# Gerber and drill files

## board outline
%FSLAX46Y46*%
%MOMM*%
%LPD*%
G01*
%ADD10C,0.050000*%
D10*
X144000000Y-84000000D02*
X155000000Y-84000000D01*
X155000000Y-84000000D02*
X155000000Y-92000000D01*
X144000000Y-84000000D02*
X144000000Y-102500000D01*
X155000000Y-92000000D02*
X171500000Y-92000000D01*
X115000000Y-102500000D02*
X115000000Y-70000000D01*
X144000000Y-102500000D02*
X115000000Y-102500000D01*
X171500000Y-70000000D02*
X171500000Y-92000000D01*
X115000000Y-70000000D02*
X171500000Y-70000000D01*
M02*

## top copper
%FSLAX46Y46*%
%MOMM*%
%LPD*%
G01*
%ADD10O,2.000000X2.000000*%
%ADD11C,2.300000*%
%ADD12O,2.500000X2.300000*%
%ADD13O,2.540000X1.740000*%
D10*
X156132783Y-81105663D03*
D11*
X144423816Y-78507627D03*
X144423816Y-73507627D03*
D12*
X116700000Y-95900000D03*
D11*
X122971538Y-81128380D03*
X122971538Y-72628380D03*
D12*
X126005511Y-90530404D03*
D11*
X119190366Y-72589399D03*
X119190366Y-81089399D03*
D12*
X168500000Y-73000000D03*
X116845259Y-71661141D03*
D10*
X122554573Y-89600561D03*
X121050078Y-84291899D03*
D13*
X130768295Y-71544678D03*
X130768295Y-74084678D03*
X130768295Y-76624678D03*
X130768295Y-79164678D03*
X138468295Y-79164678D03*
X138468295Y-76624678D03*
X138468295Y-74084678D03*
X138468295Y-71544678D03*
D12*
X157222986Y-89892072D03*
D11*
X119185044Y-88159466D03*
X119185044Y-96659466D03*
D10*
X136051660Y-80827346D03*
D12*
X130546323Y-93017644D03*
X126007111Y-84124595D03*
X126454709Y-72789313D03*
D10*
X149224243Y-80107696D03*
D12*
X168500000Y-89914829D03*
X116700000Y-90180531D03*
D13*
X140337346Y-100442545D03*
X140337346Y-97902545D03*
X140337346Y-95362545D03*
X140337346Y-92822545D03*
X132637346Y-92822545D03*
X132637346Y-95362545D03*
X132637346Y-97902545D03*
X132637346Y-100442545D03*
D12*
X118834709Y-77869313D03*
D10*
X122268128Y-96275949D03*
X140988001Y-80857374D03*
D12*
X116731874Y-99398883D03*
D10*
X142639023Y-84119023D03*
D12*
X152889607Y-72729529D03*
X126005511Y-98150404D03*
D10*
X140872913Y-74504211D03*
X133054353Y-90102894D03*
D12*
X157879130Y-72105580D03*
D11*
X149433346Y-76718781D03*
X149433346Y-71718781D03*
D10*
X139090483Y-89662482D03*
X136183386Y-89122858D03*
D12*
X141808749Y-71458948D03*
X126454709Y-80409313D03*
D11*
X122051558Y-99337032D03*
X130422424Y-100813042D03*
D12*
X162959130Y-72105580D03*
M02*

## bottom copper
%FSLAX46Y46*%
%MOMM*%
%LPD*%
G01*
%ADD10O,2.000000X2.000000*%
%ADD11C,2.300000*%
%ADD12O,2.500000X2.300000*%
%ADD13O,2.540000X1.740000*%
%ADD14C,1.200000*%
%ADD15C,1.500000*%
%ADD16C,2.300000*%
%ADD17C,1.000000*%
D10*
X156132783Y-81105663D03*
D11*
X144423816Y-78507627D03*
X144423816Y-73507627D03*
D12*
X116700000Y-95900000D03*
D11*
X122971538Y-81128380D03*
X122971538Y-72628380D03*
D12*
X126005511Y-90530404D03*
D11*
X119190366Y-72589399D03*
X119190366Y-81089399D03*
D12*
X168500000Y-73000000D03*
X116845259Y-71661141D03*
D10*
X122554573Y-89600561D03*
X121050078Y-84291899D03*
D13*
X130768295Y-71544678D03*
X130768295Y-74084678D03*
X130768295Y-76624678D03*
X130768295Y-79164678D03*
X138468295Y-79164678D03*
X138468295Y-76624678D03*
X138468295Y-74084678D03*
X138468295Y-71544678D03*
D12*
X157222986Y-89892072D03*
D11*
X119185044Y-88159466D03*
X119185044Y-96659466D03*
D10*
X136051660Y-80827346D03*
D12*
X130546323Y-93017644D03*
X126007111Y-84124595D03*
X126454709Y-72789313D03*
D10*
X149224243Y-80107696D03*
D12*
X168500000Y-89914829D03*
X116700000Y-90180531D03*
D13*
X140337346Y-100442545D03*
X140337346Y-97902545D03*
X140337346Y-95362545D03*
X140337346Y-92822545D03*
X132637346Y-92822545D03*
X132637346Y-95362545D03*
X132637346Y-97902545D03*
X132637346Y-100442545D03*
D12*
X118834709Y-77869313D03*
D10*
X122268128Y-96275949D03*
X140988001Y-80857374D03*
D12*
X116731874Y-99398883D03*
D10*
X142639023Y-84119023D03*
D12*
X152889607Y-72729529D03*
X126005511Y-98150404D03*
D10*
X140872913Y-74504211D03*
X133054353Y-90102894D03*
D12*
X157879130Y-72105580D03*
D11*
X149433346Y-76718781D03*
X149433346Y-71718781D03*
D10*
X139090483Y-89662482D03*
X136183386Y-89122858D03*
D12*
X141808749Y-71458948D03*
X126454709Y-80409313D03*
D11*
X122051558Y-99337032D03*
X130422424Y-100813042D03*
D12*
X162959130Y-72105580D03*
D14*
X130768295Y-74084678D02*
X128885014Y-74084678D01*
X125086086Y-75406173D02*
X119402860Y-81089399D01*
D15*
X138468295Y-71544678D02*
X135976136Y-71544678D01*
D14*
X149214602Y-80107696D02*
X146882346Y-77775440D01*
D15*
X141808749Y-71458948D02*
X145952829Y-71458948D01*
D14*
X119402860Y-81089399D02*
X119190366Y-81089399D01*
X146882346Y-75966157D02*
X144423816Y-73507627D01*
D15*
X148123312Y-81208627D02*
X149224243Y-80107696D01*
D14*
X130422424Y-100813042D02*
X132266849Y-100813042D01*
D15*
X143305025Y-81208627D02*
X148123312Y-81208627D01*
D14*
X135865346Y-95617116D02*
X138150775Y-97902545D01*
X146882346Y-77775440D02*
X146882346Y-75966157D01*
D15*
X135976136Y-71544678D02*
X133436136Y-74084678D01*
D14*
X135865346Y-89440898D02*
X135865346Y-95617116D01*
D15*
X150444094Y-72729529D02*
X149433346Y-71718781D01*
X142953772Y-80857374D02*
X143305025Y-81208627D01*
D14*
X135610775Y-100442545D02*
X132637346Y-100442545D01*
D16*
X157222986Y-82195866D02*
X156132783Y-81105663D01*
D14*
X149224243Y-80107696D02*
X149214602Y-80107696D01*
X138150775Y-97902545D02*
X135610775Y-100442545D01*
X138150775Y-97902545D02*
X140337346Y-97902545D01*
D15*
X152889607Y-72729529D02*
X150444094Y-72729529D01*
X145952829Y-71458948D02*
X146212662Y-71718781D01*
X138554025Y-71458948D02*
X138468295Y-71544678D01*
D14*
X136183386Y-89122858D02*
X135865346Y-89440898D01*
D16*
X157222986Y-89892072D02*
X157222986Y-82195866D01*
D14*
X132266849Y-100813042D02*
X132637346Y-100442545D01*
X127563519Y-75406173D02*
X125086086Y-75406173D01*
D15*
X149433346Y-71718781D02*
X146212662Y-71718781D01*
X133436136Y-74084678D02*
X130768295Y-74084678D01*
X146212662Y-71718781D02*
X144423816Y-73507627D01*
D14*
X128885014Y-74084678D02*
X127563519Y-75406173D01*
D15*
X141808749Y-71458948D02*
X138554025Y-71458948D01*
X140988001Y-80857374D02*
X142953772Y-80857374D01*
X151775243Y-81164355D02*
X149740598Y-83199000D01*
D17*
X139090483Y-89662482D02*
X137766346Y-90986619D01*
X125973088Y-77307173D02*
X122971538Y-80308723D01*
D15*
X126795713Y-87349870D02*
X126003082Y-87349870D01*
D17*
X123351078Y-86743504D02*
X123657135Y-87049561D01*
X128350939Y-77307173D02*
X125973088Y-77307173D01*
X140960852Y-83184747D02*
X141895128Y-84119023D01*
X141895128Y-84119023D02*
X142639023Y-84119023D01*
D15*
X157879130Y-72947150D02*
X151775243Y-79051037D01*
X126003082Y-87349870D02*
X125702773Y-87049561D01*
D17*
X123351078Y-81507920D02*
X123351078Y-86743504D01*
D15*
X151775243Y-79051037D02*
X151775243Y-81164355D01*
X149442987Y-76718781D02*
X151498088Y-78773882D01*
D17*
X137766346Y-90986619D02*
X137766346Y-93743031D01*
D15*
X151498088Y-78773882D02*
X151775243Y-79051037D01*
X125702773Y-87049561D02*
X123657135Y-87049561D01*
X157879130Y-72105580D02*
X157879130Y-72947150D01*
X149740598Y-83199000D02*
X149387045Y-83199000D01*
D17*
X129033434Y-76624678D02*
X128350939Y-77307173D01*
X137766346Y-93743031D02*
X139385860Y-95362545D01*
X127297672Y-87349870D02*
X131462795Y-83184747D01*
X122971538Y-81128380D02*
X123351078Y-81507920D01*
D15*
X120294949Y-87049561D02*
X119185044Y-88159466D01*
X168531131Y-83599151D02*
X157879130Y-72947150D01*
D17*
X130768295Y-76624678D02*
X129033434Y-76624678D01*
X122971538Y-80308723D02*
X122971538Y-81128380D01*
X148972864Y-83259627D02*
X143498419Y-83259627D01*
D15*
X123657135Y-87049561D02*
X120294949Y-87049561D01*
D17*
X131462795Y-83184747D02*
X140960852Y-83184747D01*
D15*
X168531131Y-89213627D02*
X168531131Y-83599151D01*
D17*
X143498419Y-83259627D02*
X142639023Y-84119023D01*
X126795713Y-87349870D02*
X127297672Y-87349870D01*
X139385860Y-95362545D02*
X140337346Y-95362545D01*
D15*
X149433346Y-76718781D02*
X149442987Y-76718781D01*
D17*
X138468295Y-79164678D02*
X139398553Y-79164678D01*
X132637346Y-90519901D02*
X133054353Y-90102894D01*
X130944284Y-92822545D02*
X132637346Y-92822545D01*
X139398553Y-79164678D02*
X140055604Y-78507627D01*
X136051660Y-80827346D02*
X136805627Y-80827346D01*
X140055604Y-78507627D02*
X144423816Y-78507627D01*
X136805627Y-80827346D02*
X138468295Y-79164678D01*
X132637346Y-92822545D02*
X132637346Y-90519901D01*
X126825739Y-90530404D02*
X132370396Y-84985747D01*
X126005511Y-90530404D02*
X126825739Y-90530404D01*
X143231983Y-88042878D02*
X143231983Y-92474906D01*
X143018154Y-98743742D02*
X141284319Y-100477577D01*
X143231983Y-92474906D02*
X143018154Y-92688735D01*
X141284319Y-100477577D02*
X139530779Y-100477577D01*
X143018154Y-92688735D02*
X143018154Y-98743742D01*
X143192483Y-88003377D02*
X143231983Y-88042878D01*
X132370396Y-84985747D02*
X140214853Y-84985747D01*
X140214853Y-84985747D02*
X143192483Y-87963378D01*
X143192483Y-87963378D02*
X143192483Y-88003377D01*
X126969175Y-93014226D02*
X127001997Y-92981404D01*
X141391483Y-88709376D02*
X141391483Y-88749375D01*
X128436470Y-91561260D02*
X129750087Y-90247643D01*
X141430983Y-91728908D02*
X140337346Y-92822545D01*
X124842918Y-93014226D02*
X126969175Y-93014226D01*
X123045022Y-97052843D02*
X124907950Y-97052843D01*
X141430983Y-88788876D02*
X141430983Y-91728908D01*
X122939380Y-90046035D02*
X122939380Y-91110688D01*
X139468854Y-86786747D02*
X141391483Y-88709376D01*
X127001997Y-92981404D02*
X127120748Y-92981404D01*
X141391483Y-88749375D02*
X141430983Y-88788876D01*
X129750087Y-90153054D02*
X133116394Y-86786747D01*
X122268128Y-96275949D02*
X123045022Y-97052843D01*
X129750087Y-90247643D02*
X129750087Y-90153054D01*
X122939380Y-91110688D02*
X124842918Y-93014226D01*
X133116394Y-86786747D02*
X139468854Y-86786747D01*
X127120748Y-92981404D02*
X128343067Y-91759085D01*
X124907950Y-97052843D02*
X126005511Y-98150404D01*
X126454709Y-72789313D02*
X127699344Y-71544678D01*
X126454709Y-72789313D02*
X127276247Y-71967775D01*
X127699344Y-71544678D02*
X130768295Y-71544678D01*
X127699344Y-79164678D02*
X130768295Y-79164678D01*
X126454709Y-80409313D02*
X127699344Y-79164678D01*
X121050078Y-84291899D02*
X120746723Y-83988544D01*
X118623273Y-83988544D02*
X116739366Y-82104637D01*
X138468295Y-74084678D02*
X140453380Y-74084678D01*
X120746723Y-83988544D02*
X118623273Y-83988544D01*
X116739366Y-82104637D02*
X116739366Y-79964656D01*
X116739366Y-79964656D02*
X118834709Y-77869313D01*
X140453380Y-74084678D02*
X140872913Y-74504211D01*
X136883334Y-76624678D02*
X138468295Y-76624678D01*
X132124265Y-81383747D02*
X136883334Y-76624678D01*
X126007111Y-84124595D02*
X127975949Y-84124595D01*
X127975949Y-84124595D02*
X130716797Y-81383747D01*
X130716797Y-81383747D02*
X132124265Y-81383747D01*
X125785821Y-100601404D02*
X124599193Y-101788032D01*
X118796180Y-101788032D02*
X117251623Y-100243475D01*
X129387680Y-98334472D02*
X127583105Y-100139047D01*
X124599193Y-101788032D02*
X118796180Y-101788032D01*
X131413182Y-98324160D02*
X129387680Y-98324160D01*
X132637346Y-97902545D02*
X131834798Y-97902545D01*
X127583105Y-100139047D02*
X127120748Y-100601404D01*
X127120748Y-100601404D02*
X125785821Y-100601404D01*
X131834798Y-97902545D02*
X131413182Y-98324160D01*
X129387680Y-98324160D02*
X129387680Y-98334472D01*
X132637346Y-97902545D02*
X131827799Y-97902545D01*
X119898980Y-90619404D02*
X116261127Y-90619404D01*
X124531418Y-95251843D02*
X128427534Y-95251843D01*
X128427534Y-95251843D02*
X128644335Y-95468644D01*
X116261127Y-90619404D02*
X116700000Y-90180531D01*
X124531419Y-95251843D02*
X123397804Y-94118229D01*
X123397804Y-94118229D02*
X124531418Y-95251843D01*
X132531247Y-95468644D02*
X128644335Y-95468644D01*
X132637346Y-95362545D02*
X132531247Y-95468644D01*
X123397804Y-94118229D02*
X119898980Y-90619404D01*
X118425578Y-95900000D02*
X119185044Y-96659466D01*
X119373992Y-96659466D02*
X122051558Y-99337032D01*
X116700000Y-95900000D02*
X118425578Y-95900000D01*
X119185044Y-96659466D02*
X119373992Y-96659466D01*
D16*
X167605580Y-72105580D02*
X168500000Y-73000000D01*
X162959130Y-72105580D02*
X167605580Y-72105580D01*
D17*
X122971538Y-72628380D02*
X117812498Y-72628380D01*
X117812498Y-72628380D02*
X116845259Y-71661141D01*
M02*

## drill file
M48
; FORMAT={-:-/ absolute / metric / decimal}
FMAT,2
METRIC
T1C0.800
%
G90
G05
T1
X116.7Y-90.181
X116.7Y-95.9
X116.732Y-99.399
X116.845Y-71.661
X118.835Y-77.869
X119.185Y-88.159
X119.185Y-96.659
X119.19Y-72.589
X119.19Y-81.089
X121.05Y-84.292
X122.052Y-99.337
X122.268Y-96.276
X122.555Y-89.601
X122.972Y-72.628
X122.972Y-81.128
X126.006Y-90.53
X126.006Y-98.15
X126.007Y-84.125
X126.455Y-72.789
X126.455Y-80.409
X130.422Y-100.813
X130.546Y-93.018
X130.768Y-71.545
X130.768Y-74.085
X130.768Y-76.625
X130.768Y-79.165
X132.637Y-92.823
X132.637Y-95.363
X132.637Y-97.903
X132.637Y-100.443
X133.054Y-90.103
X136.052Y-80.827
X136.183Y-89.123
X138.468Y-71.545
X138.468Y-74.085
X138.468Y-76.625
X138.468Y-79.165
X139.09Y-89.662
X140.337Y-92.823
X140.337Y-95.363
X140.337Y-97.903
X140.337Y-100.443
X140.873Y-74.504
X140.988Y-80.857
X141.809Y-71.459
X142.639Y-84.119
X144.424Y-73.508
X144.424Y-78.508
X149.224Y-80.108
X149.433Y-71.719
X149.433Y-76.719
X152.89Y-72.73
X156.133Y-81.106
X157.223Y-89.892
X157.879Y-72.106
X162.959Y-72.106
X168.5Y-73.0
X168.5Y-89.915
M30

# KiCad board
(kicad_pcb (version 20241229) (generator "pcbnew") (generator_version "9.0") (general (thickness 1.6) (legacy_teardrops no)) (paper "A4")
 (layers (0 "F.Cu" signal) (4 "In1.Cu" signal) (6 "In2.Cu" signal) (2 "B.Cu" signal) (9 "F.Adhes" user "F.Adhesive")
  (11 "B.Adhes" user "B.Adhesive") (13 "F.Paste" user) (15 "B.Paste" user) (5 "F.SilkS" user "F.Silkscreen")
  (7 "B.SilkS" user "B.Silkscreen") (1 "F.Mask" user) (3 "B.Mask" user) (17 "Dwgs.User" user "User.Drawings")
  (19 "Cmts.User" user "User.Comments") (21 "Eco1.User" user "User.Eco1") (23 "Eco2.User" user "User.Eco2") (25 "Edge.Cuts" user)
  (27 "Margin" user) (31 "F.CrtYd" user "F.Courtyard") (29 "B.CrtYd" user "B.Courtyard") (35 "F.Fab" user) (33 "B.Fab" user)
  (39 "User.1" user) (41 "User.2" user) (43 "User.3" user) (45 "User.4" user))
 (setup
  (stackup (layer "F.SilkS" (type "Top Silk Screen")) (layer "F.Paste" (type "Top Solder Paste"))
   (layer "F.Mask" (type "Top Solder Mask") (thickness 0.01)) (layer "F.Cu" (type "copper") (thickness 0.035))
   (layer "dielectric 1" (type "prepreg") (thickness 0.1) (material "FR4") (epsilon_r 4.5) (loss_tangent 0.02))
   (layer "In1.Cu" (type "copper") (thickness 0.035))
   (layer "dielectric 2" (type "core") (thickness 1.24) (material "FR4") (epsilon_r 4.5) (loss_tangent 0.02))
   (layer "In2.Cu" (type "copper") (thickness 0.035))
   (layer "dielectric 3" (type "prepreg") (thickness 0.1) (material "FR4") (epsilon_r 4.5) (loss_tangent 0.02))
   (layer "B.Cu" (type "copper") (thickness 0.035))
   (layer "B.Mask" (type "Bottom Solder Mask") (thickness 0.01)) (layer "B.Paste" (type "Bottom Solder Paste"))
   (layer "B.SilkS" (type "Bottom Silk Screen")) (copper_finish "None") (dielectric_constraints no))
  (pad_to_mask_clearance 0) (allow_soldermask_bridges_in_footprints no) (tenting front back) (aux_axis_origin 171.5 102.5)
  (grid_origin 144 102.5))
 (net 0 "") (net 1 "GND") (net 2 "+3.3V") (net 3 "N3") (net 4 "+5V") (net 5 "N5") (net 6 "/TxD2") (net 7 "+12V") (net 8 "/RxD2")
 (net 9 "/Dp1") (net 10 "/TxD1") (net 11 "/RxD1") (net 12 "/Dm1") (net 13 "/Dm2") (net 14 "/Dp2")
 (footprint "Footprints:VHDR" (layer "F.Cu") (at 156.132783 81.105663)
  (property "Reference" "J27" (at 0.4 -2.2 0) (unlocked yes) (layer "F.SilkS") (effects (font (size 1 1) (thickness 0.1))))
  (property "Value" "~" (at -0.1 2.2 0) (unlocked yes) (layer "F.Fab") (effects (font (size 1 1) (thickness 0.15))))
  (pad "1" thru_hole oval (at 0 0) (size 2 2) (drill 0.8) (layers "*.Cu" "*.Mask") (remove_unused_layers no) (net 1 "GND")))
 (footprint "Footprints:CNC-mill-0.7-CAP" (layer "F.Cu") (at 144.423816 76.007627)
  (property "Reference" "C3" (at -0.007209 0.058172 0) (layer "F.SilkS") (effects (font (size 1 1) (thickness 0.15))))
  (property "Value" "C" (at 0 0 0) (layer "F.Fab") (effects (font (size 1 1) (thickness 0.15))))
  (pad "1" thru_hole circle (at 0 2.5) (size 2.3 2.3) (drill 0.8) (layers "*.Cu" "*.Mask") (remove_unused_layers no) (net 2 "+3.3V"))
  (pad "2" thru_hole circle (at 0 -2.5) (size 2.3 2.3) (drill 0.8) (layers "*.Cu" "*.Mask") (remove_unused_layers no) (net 1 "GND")))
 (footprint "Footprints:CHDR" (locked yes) (layer "F.Cu") (at 116.7 95.9)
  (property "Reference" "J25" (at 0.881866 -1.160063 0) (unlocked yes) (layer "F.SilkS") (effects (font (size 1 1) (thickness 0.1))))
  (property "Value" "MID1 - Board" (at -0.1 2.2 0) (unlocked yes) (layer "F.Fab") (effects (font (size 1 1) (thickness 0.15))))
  (pad "1" thru_hole oval (at 0 0) (size 2.5 2.3) (drill 0.8) (layers "*.Cu" "*.Mask") (remove_unused_layers no) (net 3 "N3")))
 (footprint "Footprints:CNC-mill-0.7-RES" (layer "F.Cu") (at 122.971538 76.87838)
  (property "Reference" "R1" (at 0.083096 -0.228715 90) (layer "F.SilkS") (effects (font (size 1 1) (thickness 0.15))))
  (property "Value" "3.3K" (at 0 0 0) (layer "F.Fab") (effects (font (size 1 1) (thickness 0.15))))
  (pad "1" thru_hole circle (at 0 4.25) (size 2.3 2.3) (drill 0.8) (layers "*.Cu" "*.Mask") (remove_unused_layers no) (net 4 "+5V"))
  (pad "2" thru_hole circle (at 0 -4.25) (size 2.3 2.3) (drill 0.8) (layers "*.Cu" "*.Mask") (remove_unused_layers no) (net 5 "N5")))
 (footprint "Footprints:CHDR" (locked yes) (layer "F.Cu") (at 126.005511 90.530404)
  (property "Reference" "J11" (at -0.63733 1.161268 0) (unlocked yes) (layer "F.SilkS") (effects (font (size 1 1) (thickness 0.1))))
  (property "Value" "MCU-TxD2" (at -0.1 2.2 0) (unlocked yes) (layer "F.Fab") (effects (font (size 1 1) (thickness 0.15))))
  (pad "1" thru_hole oval (at 0 0) (size 2.5 2.3) (drill 0.8) (layers "*.Cu" "*.Mask") (remove_unused_layers no) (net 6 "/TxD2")))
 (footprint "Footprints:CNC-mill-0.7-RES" (layer "F.Cu") (at 119.190366 76.839399 180)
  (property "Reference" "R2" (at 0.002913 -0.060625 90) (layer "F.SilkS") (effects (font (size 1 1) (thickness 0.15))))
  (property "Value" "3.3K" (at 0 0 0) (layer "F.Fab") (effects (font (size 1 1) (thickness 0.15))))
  (pad "1" thru_hole circle (at 0 4.25 180) (size 2.3 2.3) (drill 0.8) (layers "*.Cu" "*.Mask") (remove_unused_layers no) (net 5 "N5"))
  (pad "2" thru_hole circle (at 0 -4.25 180) (size 2.3 2.3) (drill 0.8) (layers "*.Cu" "*.Mask") (remove_unused_layers no) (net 1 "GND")))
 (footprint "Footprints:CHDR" (layer "F.Cu") (at 168.5 73)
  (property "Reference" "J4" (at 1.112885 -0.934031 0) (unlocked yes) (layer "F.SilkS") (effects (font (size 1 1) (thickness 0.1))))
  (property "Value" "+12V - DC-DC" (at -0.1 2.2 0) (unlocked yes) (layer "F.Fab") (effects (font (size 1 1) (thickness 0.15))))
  (pad "1" thru_hole oval (at 0 0) (size 2.5 2.3) (drill 0.8) (layers "*.Cu" "*.Mask") (remove_unused_layers no) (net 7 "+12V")))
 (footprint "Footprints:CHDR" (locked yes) (layer "F.Cu") (at 116.845259 71.661141)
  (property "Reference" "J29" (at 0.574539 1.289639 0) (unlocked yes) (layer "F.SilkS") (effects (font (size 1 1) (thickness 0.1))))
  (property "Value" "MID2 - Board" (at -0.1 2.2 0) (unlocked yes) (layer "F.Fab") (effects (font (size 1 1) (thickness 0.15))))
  (pad "1" thru_hole oval (at 0 0) (size 2.5 2.3) (drill 0.8) (layers "*.Cu" "*.Mask") (remove_unused_layers no) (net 5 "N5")))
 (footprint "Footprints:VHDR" (layer "F.Cu") (at 122.554573 89.600561)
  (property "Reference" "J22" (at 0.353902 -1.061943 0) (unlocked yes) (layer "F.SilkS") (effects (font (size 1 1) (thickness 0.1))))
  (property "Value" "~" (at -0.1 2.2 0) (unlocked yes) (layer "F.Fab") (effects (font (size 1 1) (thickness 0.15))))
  (pad "1" thru_hole oval (at 0 0) (size 2 2) (drill 0.8) (layers "*.Cu" "*.Mask") (remove_unused_layers no) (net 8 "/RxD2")))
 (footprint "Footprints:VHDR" (layer "F.Cu") (at 121.050078 84.291899)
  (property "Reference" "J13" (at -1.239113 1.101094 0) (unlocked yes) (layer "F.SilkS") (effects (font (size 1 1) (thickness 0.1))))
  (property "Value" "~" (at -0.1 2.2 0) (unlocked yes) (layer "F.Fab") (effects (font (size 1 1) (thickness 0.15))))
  (pad "1" thru_hole oval (at 0 0) (size 2 2) (drill 0.8) (layers "*.Cu" "*.Mask") (remove_unused_layers no) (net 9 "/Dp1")))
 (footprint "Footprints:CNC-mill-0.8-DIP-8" (layer "F.Cu") (at 134.618295 75.354678 -90)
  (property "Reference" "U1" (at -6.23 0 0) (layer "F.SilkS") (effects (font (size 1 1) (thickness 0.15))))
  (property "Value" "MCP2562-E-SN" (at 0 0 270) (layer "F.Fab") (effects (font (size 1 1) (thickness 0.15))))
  (pad "1" thru_hole oval (at -3.81 3.85 270) (size 1.74 2.54) (drill 0.8) (layers "*.Cu" "*.Mask") (remove_unused_layers no)
   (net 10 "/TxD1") (thermal_bridge_angle 45))
  (pad "2" thru_hole oval (at -1.27 3.85 270) (size 1.74 2.54) (drill 0.8) (layers "*.Cu" "*.Mask") (remove_unused_layers no) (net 1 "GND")
   (thermal_bridge_angle 45))
  (pad "3" thru_hole oval (at 1.27 3.85 270) (size 1.74 2.54) (drill 0.8) (layers "*.Cu" "*.Mask") (remove_unused_layers no) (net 4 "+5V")
   (thermal_bridge_angle 45))
  (pad "4" thru_hole oval (at 3.81 3.85 270) (size 1.74 2.54) (drill 0.8) (layers "*.Cu" "*.Mask") (remove_unused_layers no)
   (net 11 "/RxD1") (thermal_bridge_angle 45))
  (pad "5" thru_hole oval (at 3.81 -3.85 270) (size 1.74 2.54) (drill 0.8) (layers "*.Cu" "*.Mask") (remove_unused_layers no)
   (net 2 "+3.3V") (thermal_bridge_angle 45))
  (pad "6" thru_hole oval (at 1.27 -3.85 270) (size 1.74 2.54) (drill 0.8) (layers "*.Cu" "*.Mask") (remove_unused_layers no)
   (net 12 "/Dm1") (thermal_bridge_angle 45))
  (pad "7" thru_hole oval (at -1.27 -3.85 270) (size 1.74 2.54) (drill 0.8) (layers "*.Cu" "*.Mask") (remove_unused_layers no)
   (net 9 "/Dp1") (thermal_bridge_angle 45))
  (pad "8" thru_hole oval (at -3.81 -3.85 270) (size 1.74 2.54) (drill 0.8) (layers "*.Cu" "*.Mask") (remove_unused_layers no) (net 1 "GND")
   (thermal_bridge_angle 45)))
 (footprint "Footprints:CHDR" (layer "F.Cu") (at 157.222986 89.892072)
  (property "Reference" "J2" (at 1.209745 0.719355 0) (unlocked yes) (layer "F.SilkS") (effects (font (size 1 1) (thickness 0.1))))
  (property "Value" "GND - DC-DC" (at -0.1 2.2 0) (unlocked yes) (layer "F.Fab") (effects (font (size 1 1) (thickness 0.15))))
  (pad "1" thru_hole oval (at 0 0) (size 2.5 2.3) (drill 0.8) (layers "*.Cu" "*.Mask") (remove_unused_layers no) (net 1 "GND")))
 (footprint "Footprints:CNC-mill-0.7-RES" (layer "F.Cu") (at 119.185044 92.409466 180)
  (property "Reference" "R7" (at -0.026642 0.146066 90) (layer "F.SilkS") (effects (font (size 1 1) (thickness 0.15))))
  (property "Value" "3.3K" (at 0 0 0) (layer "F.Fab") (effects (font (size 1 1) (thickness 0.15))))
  (pad "1" thru_hole circle (at 0 4.25 180) (size 2.3 2.3) (drill 0.8) (layers "*.Cu" "*.Mask") (remove_unused_layers no) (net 4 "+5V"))
  (pad "2" thru_hole circle (at 0 -4.25 180) (size 2.3 2.3) (drill 0.8) (layers "*.Cu" "*.Mask") (remove_unused_layers no) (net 3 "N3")))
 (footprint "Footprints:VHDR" (layer "F.Cu") (at 136.05166 80.827346)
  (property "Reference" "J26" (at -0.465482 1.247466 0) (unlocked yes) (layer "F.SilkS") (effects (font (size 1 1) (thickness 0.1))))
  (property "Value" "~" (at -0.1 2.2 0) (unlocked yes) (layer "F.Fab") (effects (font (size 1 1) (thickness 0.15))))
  (pad "1" thru_hole oval (at 0 0) (size 2 2) (drill 0.8) (layers "*.Cu" "*.Mask") (remove_unused_layers no) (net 2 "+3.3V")))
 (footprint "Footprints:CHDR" (layer "F.Cu") (at 130.546323 93.017644)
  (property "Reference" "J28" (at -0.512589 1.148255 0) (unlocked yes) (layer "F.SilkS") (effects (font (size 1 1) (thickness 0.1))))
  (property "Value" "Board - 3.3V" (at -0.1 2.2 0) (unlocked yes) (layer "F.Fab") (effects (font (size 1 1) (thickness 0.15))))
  (pad "1" thru_hole oval (at 0 0) (size 2.5 2.3) (drill 0.8) (layers "*.Cu" "*.Mask") (remove_unused_layers no) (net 2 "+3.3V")))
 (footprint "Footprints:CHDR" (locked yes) (layer "F.Cu") (at 126.007111 84.124595)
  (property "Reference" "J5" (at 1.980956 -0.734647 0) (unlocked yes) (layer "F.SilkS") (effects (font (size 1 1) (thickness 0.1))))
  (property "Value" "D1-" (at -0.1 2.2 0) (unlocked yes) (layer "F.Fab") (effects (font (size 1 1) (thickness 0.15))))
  (pad "1" thru_hole oval (at 0 0) (size 2.5 2.3) (drill 0.8) (layers "*.Cu" "*.Mask") (remove_unused_layers no) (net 12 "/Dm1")))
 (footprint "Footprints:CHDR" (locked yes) (layer "F.Cu") (at 126.454709 72.789313)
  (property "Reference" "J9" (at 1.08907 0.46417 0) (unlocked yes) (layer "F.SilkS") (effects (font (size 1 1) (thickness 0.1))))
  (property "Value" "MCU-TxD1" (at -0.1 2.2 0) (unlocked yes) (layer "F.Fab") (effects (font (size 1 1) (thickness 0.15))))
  (pad "1" thru_hole oval (at 0 0) (size 2.5 2.3) (drill 0.8) (layers "*.Cu" "*.Mask") (remove_unused_layers no) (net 10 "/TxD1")))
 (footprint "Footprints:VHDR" (layer "F.Cu") (at 149.224243 80.107696)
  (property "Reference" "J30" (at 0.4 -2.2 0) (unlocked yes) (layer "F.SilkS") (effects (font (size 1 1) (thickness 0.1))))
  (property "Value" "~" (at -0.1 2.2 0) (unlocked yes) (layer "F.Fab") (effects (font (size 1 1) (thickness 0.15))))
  (pad "1" thru_hole oval (at 0 0) (size 2 2) (drill 0.8) (layers "*.Cu" "*.Mask") (remove_unused_layers no) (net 1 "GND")))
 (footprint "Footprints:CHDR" (layer "F.Cu") (at 168.5 89.914829)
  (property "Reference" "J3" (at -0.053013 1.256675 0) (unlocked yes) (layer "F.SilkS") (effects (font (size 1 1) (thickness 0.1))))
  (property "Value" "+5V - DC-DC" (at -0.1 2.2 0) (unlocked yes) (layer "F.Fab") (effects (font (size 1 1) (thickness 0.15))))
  (pad "1" thru_hole oval (at 0 0) (size 2.5 2.3) (drill 0.8) (layers "*.Cu" "*.Mask") (remove_unused_layers no) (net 4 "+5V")))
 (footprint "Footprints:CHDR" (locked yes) (layer "F.Cu") (at 116.7 90.180531)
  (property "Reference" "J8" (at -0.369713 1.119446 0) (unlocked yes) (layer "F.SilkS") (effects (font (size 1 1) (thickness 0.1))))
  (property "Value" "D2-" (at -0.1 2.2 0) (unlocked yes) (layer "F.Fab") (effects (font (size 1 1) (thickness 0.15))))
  (pad "1" thru_hole oval (at 0 0) (size 2.5 2.3) (drill 0.8) (layers "*.Cu" "*.Mask") (remove_unused_layers no) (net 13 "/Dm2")))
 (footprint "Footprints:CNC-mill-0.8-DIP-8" (layer "F.Cu") (at 136.487346 96.632545 90)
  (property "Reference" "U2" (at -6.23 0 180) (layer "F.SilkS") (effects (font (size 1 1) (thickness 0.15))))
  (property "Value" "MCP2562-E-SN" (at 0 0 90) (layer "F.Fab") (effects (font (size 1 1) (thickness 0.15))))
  (pad "1" thru_hole oval (at -3.81 3.85 90) (size 1.74 2.54) (drill 0.8) (layers "*.Cu" "*.Mask") (remove_unused_layers no) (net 6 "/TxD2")
   (thermal_bridge_angle 45))
  (pad "2" thru_hole oval (at -1.27 3.85 90) (size 1.74 2.54) (drill 0.8) (layers "*.Cu" "*.Mask") (remove_unused_layers no) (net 1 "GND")
   (thermal_bridge_angle 45))
  (pad "3" thru_hole oval (at 1.27 3.85 90) (size 1.74 2.54) (drill 0.8) (layers "*.Cu" "*.Mask") (remove_unused_layers no) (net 4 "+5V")
   (thermal_bridge_angle 45))
  (pad "4" thru_hole oval (at 3.81 3.85 90) (size 1.74 2.54) (drill 0.8) (layers "*.Cu" "*.Mask") (remove_unused_layers no) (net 8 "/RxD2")
   (thermal_bridge_angle 45))
  (pad "5" thru_hole oval (at 3.81 -3.85 90) (size 1.74 2.54) (drill 0.8) (layers "*.Cu" "*.Mask") (remove_unused_layers no) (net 2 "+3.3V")
   (thermal_bridge_angle 45))
  (pad "6" thru_hole oval (at 1.27 -3.85 90) (size 1.74 2.54) (drill 0.8) (layers "*.Cu" "*.Mask") (remove_unused_layers no) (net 13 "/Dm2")
   (thermal_bridge_angle 45))
  (pad "7" thru_hole oval (at -1.27 -3.85 90) (size 1.74 2.54) (drill 0.8) (layers "*.Cu" "*.Mask") (remove_unused_layers no)
   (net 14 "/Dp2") (thermal_bridge_angle 45))
  (pad "8" thru_hole oval (at -3.81 -3.85 90) (size 1.74 2.54) (drill 0.8) (layers "*.Cu" "*.Mask") (remove_unused_layers no) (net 1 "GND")
   (thermal_bridge_angle 45)))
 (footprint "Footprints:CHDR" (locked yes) (layer "F.Cu") (at 118.834709 77.869313)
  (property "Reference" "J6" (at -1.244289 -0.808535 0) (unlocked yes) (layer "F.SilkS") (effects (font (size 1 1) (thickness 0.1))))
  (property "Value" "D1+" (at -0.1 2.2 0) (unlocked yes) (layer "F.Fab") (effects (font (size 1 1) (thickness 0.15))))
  (pad "1" thru_hole oval (at 0 0) (size 2.5 2.3) (drill 0.8) (layers "*.Cu" "*.Mask") (remove_unused_layers no) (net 9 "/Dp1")))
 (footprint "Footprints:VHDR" (layer "F.Cu") (at 122.268128 96.275949)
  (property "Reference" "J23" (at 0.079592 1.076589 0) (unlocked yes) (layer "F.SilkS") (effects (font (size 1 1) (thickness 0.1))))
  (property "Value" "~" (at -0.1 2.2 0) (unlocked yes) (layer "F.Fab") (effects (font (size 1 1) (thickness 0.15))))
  (pad "1" thru_hole oval (at 0 0) (size 2 2) (drill 0.8) (layers "*.Cu" "*.Mask") (remove_unused_layers no) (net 8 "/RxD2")))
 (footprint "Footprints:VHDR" (layer "F.Cu") (at 140.988001 80.857374)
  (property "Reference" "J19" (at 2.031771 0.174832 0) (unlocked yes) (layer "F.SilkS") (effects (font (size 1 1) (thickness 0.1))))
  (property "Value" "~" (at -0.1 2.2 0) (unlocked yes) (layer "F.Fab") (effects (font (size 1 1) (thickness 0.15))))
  (pad "1" thru_hole oval (at 0 0) (size 2 2) (drill 0.8) (layers "*.Cu" "*.Mask") (remove_unused_layers no) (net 1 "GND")))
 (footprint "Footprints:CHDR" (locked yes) (layer "F.Cu") (at 116.731874 99.398883)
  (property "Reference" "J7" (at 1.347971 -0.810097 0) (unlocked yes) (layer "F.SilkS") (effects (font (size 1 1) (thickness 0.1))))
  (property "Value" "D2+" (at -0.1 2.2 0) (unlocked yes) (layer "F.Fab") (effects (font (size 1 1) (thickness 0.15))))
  (pad "1" thru_hole oval (at 0 0) (size 2.5 2.3) (drill 0.8) (layers "*.Cu" "*.Mask") (remove_unused_layers no) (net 14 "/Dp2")))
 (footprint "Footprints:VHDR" (layer "F.Cu") (at 142.639023 84.119023)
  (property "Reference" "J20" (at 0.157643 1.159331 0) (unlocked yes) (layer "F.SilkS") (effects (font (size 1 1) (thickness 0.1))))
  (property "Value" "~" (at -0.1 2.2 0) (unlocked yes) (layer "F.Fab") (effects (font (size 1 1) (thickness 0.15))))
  (pad "1" thru_hole oval (at 0 0) (size 2 2) (drill 0.8) (layers "*.Cu" "*.Mask") (remove_unused_layers no) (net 4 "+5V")))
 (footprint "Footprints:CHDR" (layer "F.Cu") (at 152.889607 72.729529)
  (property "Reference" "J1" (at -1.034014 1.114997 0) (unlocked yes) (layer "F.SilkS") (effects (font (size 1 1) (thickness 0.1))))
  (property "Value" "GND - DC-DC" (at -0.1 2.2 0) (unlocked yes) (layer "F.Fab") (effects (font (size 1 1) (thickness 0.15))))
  (pad "1" thru_hole oval (at 0 0) (size 2.5 2.3) (drill 0.8) (layers "*.Cu" "*.Mask") (remove_unused_layers no) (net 1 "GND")))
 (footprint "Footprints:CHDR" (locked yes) (layer "F.Cu") (at 126.005511 98.150404)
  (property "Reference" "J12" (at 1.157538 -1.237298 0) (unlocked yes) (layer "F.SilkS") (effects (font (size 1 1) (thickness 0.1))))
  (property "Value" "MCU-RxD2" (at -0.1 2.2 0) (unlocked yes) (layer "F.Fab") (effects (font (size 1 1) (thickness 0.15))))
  (pad "1" thru_hole oval (at 0 0) (size 2.5 2.3) (drill 0.8) (layers "*.Cu" "*.Mask") (remove_unused_layers no) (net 8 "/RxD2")))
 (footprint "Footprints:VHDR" (layer "F.Cu") (at 140.872913 74.504211)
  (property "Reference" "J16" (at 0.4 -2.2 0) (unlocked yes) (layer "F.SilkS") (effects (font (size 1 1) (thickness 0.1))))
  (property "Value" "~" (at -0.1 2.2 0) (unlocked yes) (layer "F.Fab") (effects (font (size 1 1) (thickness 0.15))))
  (pad "1" thru_hole oval (at 0 0) (size 2 2) (drill 0.8) (layers "*.Cu" "*.Mask") (remove_unused_layers no) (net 9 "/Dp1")))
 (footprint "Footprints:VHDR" (layer "F.Cu") (at 133.054353 90.102894)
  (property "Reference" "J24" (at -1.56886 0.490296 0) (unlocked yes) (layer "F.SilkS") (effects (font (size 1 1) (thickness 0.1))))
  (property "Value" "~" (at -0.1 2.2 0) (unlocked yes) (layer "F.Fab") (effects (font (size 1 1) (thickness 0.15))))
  (pad "1" thru_hole oval (at 0 0) (size 2 2) (drill 0.8) (layers "*.Cu" "*.Mask") (remove_unused_layers no) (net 2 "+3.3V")))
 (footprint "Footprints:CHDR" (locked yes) (layer "F.Cu") (at 157.87913 72.10558)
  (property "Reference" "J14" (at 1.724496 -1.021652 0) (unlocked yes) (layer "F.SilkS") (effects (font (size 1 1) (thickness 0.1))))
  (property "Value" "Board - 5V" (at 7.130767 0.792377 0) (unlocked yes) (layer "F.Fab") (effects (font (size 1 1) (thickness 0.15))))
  (pad "1" thru_hole oval (at 0 0) (size 2.5 2.3) (drill 0.8) (layers "*.Cu" "*.Mask") (remove_unused_layers no) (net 4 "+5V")))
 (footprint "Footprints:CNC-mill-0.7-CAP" (layer "F.Cu") (at 149.433346 74.218781)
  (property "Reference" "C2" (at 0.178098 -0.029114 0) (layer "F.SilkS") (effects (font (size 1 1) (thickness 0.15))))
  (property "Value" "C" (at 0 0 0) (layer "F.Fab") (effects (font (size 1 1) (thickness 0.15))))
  (pad "1" thru_hole circle (at 0 2.5) (size 2.3 2.3) (drill 0.8) (layers "*.Cu" "*.Mask") (remove_unused_layers no) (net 4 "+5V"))
  (pad "2" thru_hole circle (at 0 -2.5) (size 2.3 2.3) (drill 0.8) (layers "*.Cu" "*.Mask") (remove_unused_layers no) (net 1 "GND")))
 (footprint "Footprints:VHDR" (layer "F.Cu") (at 139.090483 89.662482)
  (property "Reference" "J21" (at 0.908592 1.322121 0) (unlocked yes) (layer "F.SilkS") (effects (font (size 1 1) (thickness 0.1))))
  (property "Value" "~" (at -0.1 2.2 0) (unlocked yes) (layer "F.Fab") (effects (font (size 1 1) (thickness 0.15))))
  (pad "1" thru_hole oval (at 0 0) (size 2 2) (drill 0.8) (layers "*.Cu" "*.Mask") (remove_unused_layers no) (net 4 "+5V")))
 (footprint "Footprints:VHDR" (layer "F.Cu") (at 136.183386 89.122858)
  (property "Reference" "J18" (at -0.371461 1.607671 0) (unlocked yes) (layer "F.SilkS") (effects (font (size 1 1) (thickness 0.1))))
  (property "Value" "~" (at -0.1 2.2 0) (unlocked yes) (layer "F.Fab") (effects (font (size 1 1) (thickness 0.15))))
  (pad "1" thru_hole oval (at 0 0) (size 2 2) (drill 0.8) (layers "*.Cu" "*.Mask") (remove_unused_layers no) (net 1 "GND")))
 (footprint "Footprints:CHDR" (layer "F.Cu") (at 141.808749 71.458948)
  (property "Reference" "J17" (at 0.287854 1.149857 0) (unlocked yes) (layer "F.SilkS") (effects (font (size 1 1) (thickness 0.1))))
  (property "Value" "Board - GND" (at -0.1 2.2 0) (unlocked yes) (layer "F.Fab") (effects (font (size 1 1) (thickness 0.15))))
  (pad "1" thru_hole oval (at 0 0) (size 2.5 2.3) (drill 0.8) (layers "*.Cu" "*.Mask") (remove_unused_layers no) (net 1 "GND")))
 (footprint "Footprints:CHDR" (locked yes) (layer "F.Cu") (at 126.454709 80.409313)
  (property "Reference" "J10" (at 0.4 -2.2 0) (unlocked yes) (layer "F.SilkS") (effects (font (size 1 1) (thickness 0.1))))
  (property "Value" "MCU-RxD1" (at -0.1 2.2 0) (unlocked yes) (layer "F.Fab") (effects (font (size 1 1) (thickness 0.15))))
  (pad "1" thru_hole oval (at 0 0) (size 2.5 2.3) (drill 0.8) (layers "*.Cu" "*.Mask") (remove_unused_layers no) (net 11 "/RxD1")))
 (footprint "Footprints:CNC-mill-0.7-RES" (layer "F.Cu") (at 126.236991 100.075037 -100)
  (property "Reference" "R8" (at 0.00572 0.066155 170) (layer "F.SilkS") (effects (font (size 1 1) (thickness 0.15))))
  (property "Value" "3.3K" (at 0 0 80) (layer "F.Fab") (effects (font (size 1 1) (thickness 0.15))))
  (pad "1" thru_hole circle (at 0 4.25 260) (size 2.3 2.3) (drill 0.8) (layers "*.Cu" "*.Mask") (remove_unused_layers no) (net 3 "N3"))
  (pad "2" thru_hole circle (at 0 -4.25 260) (size 2.3 2.3) (drill 0.8) (layers "*.Cu" "*.Mask") (remove_unused_layers no) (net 1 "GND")))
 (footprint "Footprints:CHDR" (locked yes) (layer "F.Cu") (at 162.95913 72.10558)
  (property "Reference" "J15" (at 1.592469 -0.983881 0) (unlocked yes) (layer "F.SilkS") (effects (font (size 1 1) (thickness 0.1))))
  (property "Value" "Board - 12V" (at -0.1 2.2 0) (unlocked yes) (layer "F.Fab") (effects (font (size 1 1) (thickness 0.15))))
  (pad "1" thru_hole oval (at 0 0) (size 2.5 2.3) (drill 0.8) (layers "*.Cu" "*.Mask") (remove_unused_layers no) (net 7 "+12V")))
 (gr_line (start 144 84) (end 155 84) (stroke (width 0.05) (type default)) (locked yes) (layer "Edge.Cuts"))
 (gr_line (start 155 84) (end 155 92) (stroke (width 0.05) (type default)) (locked yes) (layer "Edge.Cuts"))
 (gr_line (start 144 84) (end 144 102.5) (stroke (width 0.05) (type default)) (locked yes) (layer "Edge.Cuts"))
 (gr_line (start 155 92) (end 171.5 92) (stroke (width 0.05) (type default)) (locked yes) (layer "Edge.Cuts"))
 (gr_line (start 115 102.5) (end 115 70) (stroke (width 0.05) (type default)) (locked yes) (layer "Edge.Cuts"))
 (gr_line (start 144 102.5) (end 115 102.5) (stroke (width 0.05) (type default)) (locked yes) (layer "Edge.Cuts"))
 (gr_line (start 171.5 70) (end 171.5 92) (stroke (width 0.05) (type default)) (locked yes) (layer "Edge.Cuts"))
 (gr_line (start 115 70) (end 171.5 70) (stroke (width 0.05) (type default)) (locked yes) (layer "Edge.Cuts"))
 (segment (start 130.768295 74.084678) (end 128.885014 74.084678) (width 1.2) (layer "B.Cu") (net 1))
 (segment (start 125.086086 75.406173) (end 119.40286 81.089399) (width 1.2) (layer "B.Cu") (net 1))
 (segment (start 138.468295 71.544678) (end 135.976136 71.544678) (width 1.5) (layer "B.Cu") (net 1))
 (segment (start 149.214602 80.107696) (end 146.882346 77.77544) (width 1.2) (layer "B.Cu") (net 1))
 (segment (start 141.808749 71.458948) (end 145.952829 71.458948) (width 1.5) (layer "B.Cu") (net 1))
 (segment (start 119.40286 81.089399) (end 119.190366 81.089399) (width 1.2) (layer "B.Cu") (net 1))
 (segment (start 146.882346 75.966157) (end 144.423816 73.507627) (width 1.2) (layer "B.Cu") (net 1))
 (segment (start 148.123312 81.208627) (end 149.224243 80.107696) (width 1.5) (layer "B.Cu") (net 1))
 (segment (start 130.422424 100.813042) (end 132.266849 100.813042) (width 1.2) (layer "B.Cu") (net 1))
 (segment (start 143.305025 81.208627) (end 148.123312 81.208627) (width 1.5) (layer "B.Cu") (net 1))
 (segment (start 135.865346 95.617116) (end 138.150775 97.902545) (width 1.2) (layer "B.Cu") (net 1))
 (segment (start 146.882346 77.77544) (end 146.882346 75.966157) (width 1.2) (layer "B.Cu") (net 1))
 (segment (start 135.976136 71.544678) (end 133.436136 74.084678) (width 1.5) (layer "B.Cu") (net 1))
 (segment (start 135.865346 89.440898) (end 135.865346 95.617116) (width 1.2) (layer "B.Cu") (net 1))
 (segment (start 150.444094 72.729529) (end 149.433346 71.718781) (width 1.5) (layer "B.Cu") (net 1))
 (segment (start 142.953772 80.857374) (end 143.305025 81.208627) (width 1.5) (layer "B.Cu") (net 1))
 (segment (start 135.610775 100.442545) (end 132.637346 100.442545) (width 1.2) (layer "B.Cu") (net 1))
 (segment (start 157.222986 82.195866) (end 156.132783 81.105663) (width 2.3) (layer "B.Cu") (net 1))
 (segment (start 149.224243 80.107696) (end 149.214602 80.107696) (width 1.2) (layer "B.Cu") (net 1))
 (segment (start 138.150775 97.902545) (end 135.610775 100.442545) (width 1.2) (layer "B.Cu") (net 1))
 (segment (start 138.150775 97.902545) (end 140.337346 97.902545) (width 1.2) (layer "B.Cu") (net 1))
 (segment (start 152.889607 72.729529) (end 150.444094 72.729529) (width 1.5) (layer "B.Cu") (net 1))
 (segment (start 145.952829 71.458948) (end 146.212662 71.718781) (width 1.5) (layer "B.Cu") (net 1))
 (segment (start 138.554025 71.458948) (end 138.468295 71.544678) (width 1.5) (layer "B.Cu") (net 1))
 (segment (start 136.183386 89.122858) (end 135.865346 89.440898) (width 1.2) (layer "B.Cu") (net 1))
 (segment (start 157.222986 89.892072) (end 157.222986 82.195866) (width 2.3) (layer "B.Cu") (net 1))
 (segment (start 132.266849 100.813042) (end 132.637346 100.442545) (width 1.2) (layer "B.Cu") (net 1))
 (segment (start 127.563519 75.406173) (end 125.086086 75.406173) (width 1.2) (layer "B.Cu") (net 1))
 (segment (start 149.433346 71.718781) (end 146.212662 71.718781) (width 1.5) (layer "B.Cu") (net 1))
 (segment (start 133.436136 74.084678) (end 130.768295 74.084678) (width 1.5) (layer "B.Cu") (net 1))
 (segment (start 146.212662 71.718781) (end 144.423816 73.507627) (width 1.5) (layer "B.Cu") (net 1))
 (segment (start 128.885014 74.084678) (end 127.563519 75.406173) (width 1.2) (layer "B.Cu") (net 1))
 (segment (start 141.808749 71.458948) (end 138.554025 71.458948) (width 1.5) (layer "B.Cu") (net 1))
 (segment (start 140.988001 80.857374) (end 142.953772 80.857374) (width 1.5) (layer "B.Cu") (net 1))
 (segment (start 151.775243 81.164355) (end 149.740598 83.199) (width 1.5) (layer "B.Cu") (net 4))
 (segment (start 139.090483 89.662482) (end 137.766346 90.986619) (width 1) (layer "B.Cu") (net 4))
 (segment (start 125.973088 77.307173) (end 122.971538 80.308723) (width 1) (layer "B.Cu") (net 4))
 (segment (start 126.795713 87.34987) (end 126.003082 87.34987) (width 1.5) (layer "B.Cu") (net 4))
 (segment (start 123.351078 86.743504) (end 123.657135 87.049561) (width 1) (layer "B.Cu") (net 4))
 (segment (start 128.350939 77.307173) (end 125.973088 77.307173) (width 1) (layer "B.Cu") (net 4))
 (segment (start 140.960852 83.184747) (end 141.895128 84.119023) (width 1) (layer "B.Cu") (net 4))
 (segment (start 141.895128 84.119023) (end 142.639023 84.119023) (width 1) (layer "B.Cu") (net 4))
 (segment (start 157.87913 72.94715) (end 151.775243 79.051037) (width 1.5) (layer "B.Cu") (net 4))
 (segment (start 126.003082 87.34987) (end 125.702773 87.049561) (width 1.5) (layer "B.Cu") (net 4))
 (segment (start 123.351078 81.50792) (end 123.351078 86.743504) (width 1) (layer "B.Cu") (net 4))
 (segment (start 151.775243 79.051037) (end 151.775243 81.164355) (width 1.5) (layer "B.Cu") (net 4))
 (segment (start 149.442987 76.718781) (end 151.498088 78.773882) (width 1.5) (layer "B.Cu") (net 4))
 (segment (start 137.766346 90.986619) (end 137.766346 93.743031) (width 1) (layer "B.Cu") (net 4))
 (segment (start 151.498088 78.773882) (end 151.775243 79.051037) (width 1.5) (layer "B.Cu") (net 4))
 (segment (start 125.702773 87.049561) (end 123.657135 87.049561) (width 1.5) (layer "B.Cu") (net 4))
 (segment (start 157.87913 72.10558) (end 157.87913 72.94715) (width 1.5) (layer "B.Cu") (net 4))
 (segment (start 149.740598 83.199) (end 149.387045 83.199) (width 1.5) (layer "B.Cu") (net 4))
 (segment (start 129.033434 76.624678) (end 128.350939 77.307173) (width 1) (layer "B.Cu") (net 4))
 (segment (start 137.766346 93.743031) (end 139.38586 95.362545) (width 1) (layer "B.Cu") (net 4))
 (segment (start 127.297672 87.34987) (end 131.462795 83.184747) (width 1) (layer "B.Cu") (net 4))
 (segment (start 122.971538 81.12838) (end 123.351078 81.50792) (width 1) (layer "B.Cu") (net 4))
 (segment (start 120.294949 87.049561) (end 119.185044 88.159466) (width 1.5) (layer "B.Cu") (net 4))
 (segment (start 168.531131 83.599151) (end 157.87913 72.94715) (width 1.5) (layer "B.Cu") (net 4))
 (segment (start 130.768295 76.624678) (end 129.033434 76.624678) (width 1) (layer "B.Cu") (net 4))
 (segment (start 122.971538 80.308723) (end 122.971538 81.12838) (width 1) (layer "B.Cu") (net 4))
 (segment (start 148.972864 83.259627) (end 143.498419 83.259627) (width 1) (layer "B.Cu") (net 4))
 (segment (start 123.657135 87.049561) (end 120.294949 87.049561) (width 1.5) (layer "B.Cu") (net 4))
 (segment (start 131.462795 83.184747) (end 140.960852 83.184747) (width 1) (layer "B.Cu") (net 4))
 (segment (start 168.531131 89.213627) (end 168.531131 83.599151) (width 1.5) (layer "B.Cu") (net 4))
 (segment (start 143.498419 83.259627) (end 142.639023 84.119023) (width 1) (layer "B.Cu") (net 4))
 (segment (start 126.795713 87.34987) (end 127.297672 87.34987) (width 1) (layer "B.Cu") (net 4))
 (segment (start 139.38586 95.362545) (end 140.337346 95.362545) (width 1) (layer "B.Cu") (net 4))
 (segment (start 149.433346 76.718781) (end 149.442987 76.718781) (width 1.5) (layer "B.Cu") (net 4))
 (segment (start 138.468295 79.164678) (end 139.398553 79.164678) (width 1) (layer "B.Cu") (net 2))
 (segment (start 132.637346 90.519901) (end 133.054353 90.102894) (width 1) (layer "B.Cu") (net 2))
 (segment (start 130.944284 92.822545) (end 132.637346 92.822545) (width 1) (layer "B.Cu") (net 2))
 (segment (start 139.398553 79.164678) (end 140.055604 78.507627) (width 1) (layer "B.Cu") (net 2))
 (segment (start 136.05166 80.827346) (end 136.805627 80.827346) (width 1) (layer "B.Cu") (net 2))
 (segment (start 140.055604 78.507627) (end 144.423816 78.507627) (width 1) (layer "B.Cu") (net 2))
 (segment (start 136.805627 80.827346) (end 138.468295 79.164678) (width 1) (layer "B.Cu") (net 2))
 (segment (start 132.637346 92.822545) (end 132.637346 90.519901) (width 1) (layer "B.Cu") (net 2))
 (segment (start 126.825739 90.530404) (end 132.370396 84.985747) (width 1) (layer "B.Cu") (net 6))
 (segment (start 126.005511 90.530404) (end 126.825739 90.530404) (width 1) (layer "B.Cu") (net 6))
 (segment (start 143.231983 88.042878) (end 143.231983 92.474906) (width 1) (layer "B.Cu") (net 6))
 (segment (start 143.018154 98.743742) (end 141.284319 100.477577) (width 1) (layer "B.Cu") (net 6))
 (segment (start 143.231983 92.474906) (end 143.018154 92.688735) (width 1) (layer "B.Cu") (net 6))
 (segment (start 141.284319 100.477577) (end 139.530779 100.477577) (width 1) (layer "B.Cu") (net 6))
 (segment (start 143.018154 92.688735) (end 143.018154 98.743742) (width 1) (layer "B.Cu") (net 6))
 (segment (start 143.192483 88.003377) (end 143.231983 88.042878) (width 1) (layer "B.Cu") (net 6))
 (segment (start 132.370396 84.985747) (end 140.214853 84.985747) (width 1) (layer "B.Cu") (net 6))
 (segment (start 140.214853 84.985747) (end 143.192483 87.963378) (width 1) (layer "B.Cu") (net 6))
 (segment (start 143.192483 87.963378) (end 143.192483 88.003377) (width 1) (layer "B.Cu") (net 6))
 (segment (start 126.969175 93.014226) (end 127.001997 92.981404) (width 1) (layer "B.Cu") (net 8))
 (segment (start 141.391483 88.709376) (end 141.391483 88.749375) (width 1) (layer "B.Cu") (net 8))
 (segment (start 128.43647 91.56126) (end 129.750087 90.247643) (width 1) (layer "B.Cu") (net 8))
 (segment (start 141.430983 91.728908) (end 140.337346 92.822545) (width 1) (layer "B.Cu") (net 8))
 (segment (start 124.842918 93.014226) (end 126.969175 93.014226) (width 1) (layer "B.Cu") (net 8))
 (segment (start 123.045022 97.052843) (end 124.90795 97.052843) (width 1) (layer "B.Cu") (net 8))
 (segment (start 141.430983 88.788876) (end 141.430983 91.728908) (width 1) (layer "B.Cu") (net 8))
 (segment (start 122.93938 90.046035) (end 122.93938 91.110688) (width 1) (layer "B.Cu") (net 8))
 (segment (start 139.468854 86.786747) (end 141.391483 88.709376) (width 1) (layer "B.Cu") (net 8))
 (segment (start 127.001997 92.981404) (end 127.120748 92.981404) (width 1) (layer "B.Cu") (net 8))
 (segment (start 141.391483 88.749375) (end 141.430983 88.788876) (width 1) (layer "B.Cu") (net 8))
 (segment (start 129.750087 90.153054) (end 133.116394 86.786747) (width 1) (layer "B.Cu") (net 8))
 (segment (start 122.268128 96.275949) (end 123.045022 97.052843) (width 1) (layer "B.Cu") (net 8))
 (segment (start 129.750087 90.247643) (end 129.750087 90.153054) (width 1) (layer "B.Cu") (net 8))
 (segment (start 122.93938 91.110688) (end 124.842918 93.014226) (width 1) (layer "B.Cu") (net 8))
 (segment (start 133.116394 86.786747) (end 139.468854 86.786747) (width 1) (layer "B.Cu") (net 8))
 (segment (start 127.120748 92.981404) (end 128.343067 91.759085) (width 1) (layer "B.Cu") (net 8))
 (segment (start 124.90795 97.052843) (end 126.005511 98.150404) (width 1) (layer "B.Cu") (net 8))
 (segment (start 126.454709 72.789313) (end 127.699344 71.544678) (width 1) (layer "B.Cu") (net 10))
 (segment (start 126.454709 72.789313) (end 127.276247 71.967775) (width 1) (layer "B.Cu") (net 10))
 (segment (start 127.699344 71.544678) (end 130.768295 71.544678) (width 1) (layer "B.Cu") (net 10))
 (segment (start 127.699344 79.164678) (end 130.768295 79.164678) (width 1) (layer "B.Cu") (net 11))
 (segment (start 126.454709 80.409313) (end 127.699344 79.164678) (width 1) (layer "B.Cu") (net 11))
 (segment (start 121.050078 84.291899) (end 120.746723 83.988544) (width 1) (layer "B.Cu") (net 9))
 (segment (start 118.623273 83.988544) (end 116.739366 82.104637) (width 1) (layer "B.Cu") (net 9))
 (segment (start 138.468295 74.084678) (end 140.45338 74.084678) (width 1) (layer "B.Cu") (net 9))
 (segment (start 120.746723 83.988544) (end 118.623273 83.988544) (width 1) (layer "B.Cu") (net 9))
 (segment (start 116.739366 82.104637) (end 116.739366 79.964656) (width 1) (layer "B.Cu") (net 9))
 (segment (start 116.739366 79.964656) (end 118.834709 77.869313) (width 1) (layer "B.Cu") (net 9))
 (segment (start 140.45338 74.084678) (end 140.872913 74.504211) (width 1) (layer "B.Cu") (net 9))
 (segment (start 136.883334 76.624678) (end 138.468295 76.624678) (width 1) (layer "B.Cu") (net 12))
 (segment (start 132.124265 81.383747) (end 136.883334 76.624678) (width 1) (layer "B.Cu") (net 12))
 (segment (start 126.007111 84.124595) (end 127.975949 84.124595) (width 1) (layer "B.Cu") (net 12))
 (segment (start 127.975949 84.124595) (end 130.716797 81.383747) (width 1) (layer "B.Cu") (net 12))
 (segment (start 130.716797 81.383747) (end 132.124265 81.383747) (width 1) (layer "B.Cu") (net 12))
 (segment (start 125.785821 100.601404) (end 124.599193 101.788032) (width 1) (layer "B.Cu") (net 14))
 (segment (start 118.79618 101.788032) (end 117.251623 100.243475) (width 1) (layer "B.Cu") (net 14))
 (segment (start 129.38768 98.334472) (end 127.583105 100.139047) (width 1) (layer "B.Cu") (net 14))
 (segment (start 124.599193 101.788032) (end 118.79618 101.788032) (width 1) (layer "B.Cu") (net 14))
 (segment (start 131.413182 98.32416) (end 129.38768 98.32416) (width 1) (layer "B.Cu") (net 14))
 (segment (start 132.637346 97.902545) (end 131.834798 97.902545) (width 1) (layer "B.Cu") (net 14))
 (segment (start 127.583105 100.139047) (end 127.120748 100.601404) (width 1) (layer "B.Cu") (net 14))
 (segment (start 127.120748 100.601404) (end 125.785821 100.601404) (width 1) (layer "B.Cu") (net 14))
 (segment (start 131.834798 97.902545) (end 131.413182 98.32416) (width 1) (layer "B.Cu") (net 14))
 (segment (start 129.38768 98.32416) (end 129.38768 98.334472) (width 1) (layer "B.Cu") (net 14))
 (segment (start 132.637346 97.902545) (end 131.827799 97.902545) (width 1) (layer "B.Cu") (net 14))
 (segment (start 119.89898 90.619404) (end 116.261127 90.619404) (width 1) (layer "B.Cu") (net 13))
 (segment (start 124.531418 95.251843) (end 128.427534 95.251843) (width 1) (layer "B.Cu") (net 13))
 (segment (start 128.427534 95.251843) (end 128.644335 95.468644) (width 1) (layer "B.Cu") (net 13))
 (segment (start 116.261127 90.619404) (end 116.7 90.180531) (width 1) (layer "B.Cu") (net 13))
 (segment (start 124.531419 95.251843) (end 123.397804 94.118229) (width 1) (layer "B.Cu") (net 13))
 (segment (start 123.397804 94.118229) (end 124.531418 95.251843) (width 1) (layer "B.Cu") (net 13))
 (segment (start 132.531247 95.468644) (end 128.644335 95.468644) (width 1) (layer "B.Cu") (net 13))
 (segment (start 132.637346 95.362545) (end 132.531247 95.468644) (width 1) (layer "B.Cu") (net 13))
 (segment (start 123.397804 94.118229) (end 119.89898 90.619404) (width 1) (layer "B.Cu") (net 13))
 (segment (start 118.425578 95.9) (end 119.185044 96.659466) (width 1) (layer "B.Cu") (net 3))
 (segment (start 119.373992 96.659466) (end 122.051558 99.337032) (width 1) (layer "B.Cu") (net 3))
 (segment (start 116.7 95.9) (end 118.425578 95.9) (width 1) (layer "B.Cu") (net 3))
 (segment (start 119.185044 96.659466) (end 119.373992 96.659466) (width 1) (layer "B.Cu") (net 3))
 (segment (start 167.60558 72.10558) (end 168.5 73) (width 2.3) (layer "B.Cu") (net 7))
 (segment (start 162.95913 72.10558) (end 167.60558 72.10558) (width 2.3) (layer "B.Cu") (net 7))
 (segment (start 122.971538 72.62838) (end 117.812498 72.62838) (width 1) (layer "B.Cu") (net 5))
 (segment (start 117.812498 72.62838) (end 116.845259 71.661141) (width 1) (layer "B.Cu") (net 5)))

